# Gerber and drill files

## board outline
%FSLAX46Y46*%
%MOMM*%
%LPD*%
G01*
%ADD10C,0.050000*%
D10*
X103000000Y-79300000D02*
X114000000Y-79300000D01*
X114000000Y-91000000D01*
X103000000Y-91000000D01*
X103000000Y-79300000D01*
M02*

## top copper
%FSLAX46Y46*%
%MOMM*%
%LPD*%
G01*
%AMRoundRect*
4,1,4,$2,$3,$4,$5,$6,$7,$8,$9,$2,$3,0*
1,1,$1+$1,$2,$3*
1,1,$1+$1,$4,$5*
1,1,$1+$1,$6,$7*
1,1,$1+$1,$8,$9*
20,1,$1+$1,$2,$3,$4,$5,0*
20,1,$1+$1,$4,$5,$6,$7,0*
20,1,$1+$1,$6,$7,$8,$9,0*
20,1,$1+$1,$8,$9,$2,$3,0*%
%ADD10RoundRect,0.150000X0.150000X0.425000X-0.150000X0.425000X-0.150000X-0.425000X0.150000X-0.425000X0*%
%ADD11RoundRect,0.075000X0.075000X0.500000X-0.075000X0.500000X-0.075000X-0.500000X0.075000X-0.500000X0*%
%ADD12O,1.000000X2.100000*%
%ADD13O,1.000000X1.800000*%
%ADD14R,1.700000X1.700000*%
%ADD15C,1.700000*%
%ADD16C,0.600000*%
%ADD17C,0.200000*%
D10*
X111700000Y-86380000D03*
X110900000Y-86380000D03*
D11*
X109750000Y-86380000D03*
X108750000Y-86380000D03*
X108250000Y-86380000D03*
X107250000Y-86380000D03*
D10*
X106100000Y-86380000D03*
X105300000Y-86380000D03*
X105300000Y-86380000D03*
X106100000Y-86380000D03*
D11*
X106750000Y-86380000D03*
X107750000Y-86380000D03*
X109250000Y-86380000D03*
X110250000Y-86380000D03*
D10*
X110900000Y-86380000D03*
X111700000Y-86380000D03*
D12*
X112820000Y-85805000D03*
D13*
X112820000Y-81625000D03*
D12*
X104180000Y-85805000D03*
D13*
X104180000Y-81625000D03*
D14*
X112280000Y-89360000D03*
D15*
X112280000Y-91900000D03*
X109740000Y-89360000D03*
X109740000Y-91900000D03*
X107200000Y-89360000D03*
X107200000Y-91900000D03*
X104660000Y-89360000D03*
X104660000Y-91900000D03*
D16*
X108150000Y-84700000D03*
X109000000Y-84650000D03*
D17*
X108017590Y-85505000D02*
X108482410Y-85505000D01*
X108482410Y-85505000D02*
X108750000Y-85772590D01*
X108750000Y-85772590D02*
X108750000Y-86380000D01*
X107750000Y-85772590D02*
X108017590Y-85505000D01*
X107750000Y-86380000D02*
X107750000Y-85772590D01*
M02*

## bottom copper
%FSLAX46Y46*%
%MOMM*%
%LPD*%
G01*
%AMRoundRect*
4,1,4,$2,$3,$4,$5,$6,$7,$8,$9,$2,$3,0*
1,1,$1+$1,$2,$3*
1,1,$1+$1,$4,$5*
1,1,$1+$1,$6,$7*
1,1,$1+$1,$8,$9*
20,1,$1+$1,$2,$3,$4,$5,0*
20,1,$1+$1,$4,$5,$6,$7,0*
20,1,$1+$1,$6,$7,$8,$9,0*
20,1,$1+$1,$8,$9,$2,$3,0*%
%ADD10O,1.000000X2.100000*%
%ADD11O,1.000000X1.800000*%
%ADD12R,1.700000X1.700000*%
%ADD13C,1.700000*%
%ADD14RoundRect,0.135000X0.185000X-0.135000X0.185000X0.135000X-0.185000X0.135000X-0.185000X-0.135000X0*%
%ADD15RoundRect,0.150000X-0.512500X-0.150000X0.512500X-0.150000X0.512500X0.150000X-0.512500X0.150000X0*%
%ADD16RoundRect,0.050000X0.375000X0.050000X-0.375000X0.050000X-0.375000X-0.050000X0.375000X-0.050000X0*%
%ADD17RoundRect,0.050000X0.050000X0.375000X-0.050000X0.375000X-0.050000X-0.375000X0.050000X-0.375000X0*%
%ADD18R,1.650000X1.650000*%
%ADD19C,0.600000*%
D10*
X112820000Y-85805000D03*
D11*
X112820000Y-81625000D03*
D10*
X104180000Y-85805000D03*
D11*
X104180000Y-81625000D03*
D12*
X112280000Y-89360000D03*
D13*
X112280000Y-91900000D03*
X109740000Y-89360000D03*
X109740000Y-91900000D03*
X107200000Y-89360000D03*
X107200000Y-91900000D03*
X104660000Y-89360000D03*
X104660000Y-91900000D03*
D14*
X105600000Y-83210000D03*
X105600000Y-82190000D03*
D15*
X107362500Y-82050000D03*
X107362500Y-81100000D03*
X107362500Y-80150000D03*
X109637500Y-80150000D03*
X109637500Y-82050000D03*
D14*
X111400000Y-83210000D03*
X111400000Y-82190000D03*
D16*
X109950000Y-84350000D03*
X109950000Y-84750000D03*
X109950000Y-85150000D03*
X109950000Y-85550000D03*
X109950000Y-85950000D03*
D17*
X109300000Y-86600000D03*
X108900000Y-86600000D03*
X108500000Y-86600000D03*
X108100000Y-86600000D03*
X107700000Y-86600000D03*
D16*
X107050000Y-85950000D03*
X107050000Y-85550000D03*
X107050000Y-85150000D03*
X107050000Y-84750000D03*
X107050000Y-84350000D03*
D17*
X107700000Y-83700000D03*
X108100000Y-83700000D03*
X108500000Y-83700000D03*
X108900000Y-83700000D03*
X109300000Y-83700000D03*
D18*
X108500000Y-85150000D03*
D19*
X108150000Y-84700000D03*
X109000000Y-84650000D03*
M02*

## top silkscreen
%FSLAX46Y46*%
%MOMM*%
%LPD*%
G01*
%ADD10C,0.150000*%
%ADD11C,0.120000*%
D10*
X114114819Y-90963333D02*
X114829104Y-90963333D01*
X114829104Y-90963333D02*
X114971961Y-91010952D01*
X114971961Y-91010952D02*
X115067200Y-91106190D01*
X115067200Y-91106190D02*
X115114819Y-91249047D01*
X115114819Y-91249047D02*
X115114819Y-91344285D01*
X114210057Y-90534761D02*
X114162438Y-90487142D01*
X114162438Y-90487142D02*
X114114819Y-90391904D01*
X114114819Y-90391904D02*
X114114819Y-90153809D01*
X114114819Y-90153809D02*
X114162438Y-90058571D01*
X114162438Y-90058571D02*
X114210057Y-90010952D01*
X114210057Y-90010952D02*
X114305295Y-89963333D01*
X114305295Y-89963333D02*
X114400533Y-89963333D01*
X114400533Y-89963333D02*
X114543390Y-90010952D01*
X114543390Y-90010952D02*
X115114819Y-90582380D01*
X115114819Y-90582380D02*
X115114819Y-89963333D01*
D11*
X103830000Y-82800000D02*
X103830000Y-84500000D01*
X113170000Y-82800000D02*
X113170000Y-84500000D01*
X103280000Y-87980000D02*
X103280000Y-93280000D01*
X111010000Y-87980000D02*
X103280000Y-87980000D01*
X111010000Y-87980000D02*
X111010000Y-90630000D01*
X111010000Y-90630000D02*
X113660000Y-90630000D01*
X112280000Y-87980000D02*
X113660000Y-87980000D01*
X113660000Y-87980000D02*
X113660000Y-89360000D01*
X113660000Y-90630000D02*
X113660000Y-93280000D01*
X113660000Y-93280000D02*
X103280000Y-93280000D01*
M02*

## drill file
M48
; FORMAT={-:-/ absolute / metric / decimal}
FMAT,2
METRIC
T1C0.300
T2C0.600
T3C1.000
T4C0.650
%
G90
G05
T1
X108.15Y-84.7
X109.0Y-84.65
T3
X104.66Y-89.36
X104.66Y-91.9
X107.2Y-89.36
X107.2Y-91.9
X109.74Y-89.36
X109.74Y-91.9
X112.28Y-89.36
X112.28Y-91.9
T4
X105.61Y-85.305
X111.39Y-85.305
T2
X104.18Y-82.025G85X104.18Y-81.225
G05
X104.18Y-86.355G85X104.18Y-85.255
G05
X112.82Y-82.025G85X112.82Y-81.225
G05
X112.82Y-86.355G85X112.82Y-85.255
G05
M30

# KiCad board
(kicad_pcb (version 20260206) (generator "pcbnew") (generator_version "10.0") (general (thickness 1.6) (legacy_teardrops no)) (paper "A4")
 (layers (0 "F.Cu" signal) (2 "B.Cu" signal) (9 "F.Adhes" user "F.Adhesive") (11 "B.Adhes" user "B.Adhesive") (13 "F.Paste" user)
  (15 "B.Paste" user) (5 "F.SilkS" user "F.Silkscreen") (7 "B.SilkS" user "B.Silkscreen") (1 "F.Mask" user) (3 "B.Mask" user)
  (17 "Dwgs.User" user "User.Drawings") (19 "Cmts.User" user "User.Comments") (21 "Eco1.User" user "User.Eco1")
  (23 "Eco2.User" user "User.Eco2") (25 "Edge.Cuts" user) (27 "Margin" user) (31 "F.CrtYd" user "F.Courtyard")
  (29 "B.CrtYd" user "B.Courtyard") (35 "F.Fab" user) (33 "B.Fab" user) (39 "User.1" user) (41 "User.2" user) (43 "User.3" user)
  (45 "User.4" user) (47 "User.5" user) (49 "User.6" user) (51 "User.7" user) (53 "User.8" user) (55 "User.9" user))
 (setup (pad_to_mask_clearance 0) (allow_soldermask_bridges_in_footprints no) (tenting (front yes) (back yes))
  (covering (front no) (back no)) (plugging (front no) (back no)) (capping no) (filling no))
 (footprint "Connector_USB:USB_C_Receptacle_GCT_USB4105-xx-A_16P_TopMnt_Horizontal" (layer "F.Cu") (at 108.5 82.7 180)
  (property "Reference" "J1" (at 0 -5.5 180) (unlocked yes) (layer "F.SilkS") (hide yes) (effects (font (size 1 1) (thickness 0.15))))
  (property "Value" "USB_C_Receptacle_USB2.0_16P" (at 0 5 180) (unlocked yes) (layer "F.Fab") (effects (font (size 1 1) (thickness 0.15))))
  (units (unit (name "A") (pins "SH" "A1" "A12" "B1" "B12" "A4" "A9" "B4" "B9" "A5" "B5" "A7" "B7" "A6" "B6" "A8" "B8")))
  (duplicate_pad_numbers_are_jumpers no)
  (fp_line (start 4.67 -0.1) (end 4.67 -1.8) (stroke (width 0.12) (type solid)) (layer "F.SilkS"))
  (fp_line (start -4.67 -0.1) (end -4.67 -1.8) (stroke (width 0.12) (type solid)) (layer "F.SilkS"))
  (pad "" np_thru_hole circle (at -2.89 -2.605 180) (size 0.65 0.65) (drill 0.65) (layers "*.Cu" "*.Mask"))
  (pad "" np_thru_hole circle (at 2.89 -2.605 180) (size 0.65 0.65) (drill 0.65) (layers "*.Cu" "*.Mask"))
  (pad "A1" smd roundrect (at -3.2 -3.68 180) (size 0.6 1.15) (layers "F.Cu" "F.Mask" "F.Paste") (roundrect_rratio 0.25) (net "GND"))
  (pad "A4" smd roundrect (at -2.4 -3.68 180) (size 0.6 1.15) (layers "F.Cu" "F.Mask" "F.Paste") (roundrect_rratio 0.25) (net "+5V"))
  (pad "A5" smd roundrect (at -1.25 -3.68 180) (size 0.3 1.15) (layers "F.Cu" "F.Mask" "F.Paste") (roundrect_rratio 0.25)
   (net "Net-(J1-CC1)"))
  (pad "A6" smd roundrect (at -0.25 -3.68 180) (size 0.3 1.15) (layers "F.Cu" "F.Mask" "F.Paste") (roundrect_rratio 0.25) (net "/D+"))
  (pad "A7" smd roundrect (at 0.25 -3.68 180) (size 0.3 1.15) (layers "F.Cu" "F.Mask" "F.Paste") (roundrect_rratio 0.25) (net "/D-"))
  (pad "A8" smd roundrect (at 1.25 -3.68 180) (size 0.3 1.15) (layers "F.Cu" "F.Mask" "F.Paste") (roundrect_rratio 0.25)
   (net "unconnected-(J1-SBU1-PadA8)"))
  (pad "A9" smd roundrect (at 2.4 -3.68 180) (size 0.6 1.15) (layers "F.Cu" "F.Mask" "F.Paste") (roundrect_rratio 0.25) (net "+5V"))
  (pad "A12" smd roundrect (at 3.2 -3.68 180) (size 0.6 1.15) (layers "F.Cu" "F.Mask" "F.Paste") (roundrect_rratio 0.25) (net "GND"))
  (pad "B1" smd roundrect (at 3.2 -3.68 180) (size 0.6 1.15) (layers "F.Cu" "F.Mask" "F.Paste") (roundrect_rratio 0.25) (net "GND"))
  (pad "B4" smd roundrect (at 2.4 -3.68 180) (size 0.6 1.15) (layers "F.Cu" "F.Mask" "F.Paste") (roundrect_rratio 0.25) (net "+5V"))
  (pad "B5" smd roundrect (at 1.75 -3.68 180) (size 0.3 1.15) (layers "F.Cu" "F.Mask" "F.Paste") (roundrect_rratio 0.25)
   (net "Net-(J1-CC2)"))
  (pad "B6" smd roundrect (at 0.75 -3.68 180) (size 0.3 1.15) (layers "F.Cu" "F.Mask" "F.Paste") (roundrect_rratio 0.25) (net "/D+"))
  (pad "B7" smd roundrect (at -0.75 -3.68 180) (size 0.3 1.15) (layers "F.Cu" "F.Mask" "F.Paste") (roundrect_rratio 0.25) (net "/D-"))
  (pad "B8" smd roundrect (at -1.75 -3.68 180) (size 0.3 1.15) (layers "F.Cu" "F.Mask" "F.Paste") (roundrect_rratio 0.25)
   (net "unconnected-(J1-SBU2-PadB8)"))
  (pad "B9" smd roundrect (at -2.4 -3.68 180) (size 0.6 1.15) (layers "F.Cu" "F.Mask" "F.Paste") (roundrect_rratio 0.25) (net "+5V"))
  (pad "B12" smd roundrect (at -3.2 -3.68 180) (size 0.6 1.15) (layers "F.Cu" "F.Mask" "F.Paste") (roundrect_rratio 0.25) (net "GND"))
  (pad "SH" thru_hole oval (at -4.32 -3.105 180) (size 1 2.1) (drill oval 0.6 1.7) (layers "*.Cu" "*.Mask" "F.Paste")
   (remove_unused_layers no) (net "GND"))
  (pad "SH" thru_hole oval (at -4.32 1.075 180) (size 1 1.8) (drill oval 0.6 1.4) (layers "*.Cu" "*.Mask" "F.Paste")
   (remove_unused_layers no) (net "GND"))
  (pad "SH" thru_hole oval (at 4.32 -3.105 180) (size 1 2.1) (drill oval 0.6 1.7) (layers "*.Cu" "*.Mask" "F.Paste")
   (remove_unused_layers no) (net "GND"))
  (pad "SH" thru_hole oval (at 4.32 1.075 180) (size 1 1.8) (drill oval 0.6 1.4) (layers "*.Cu" "*.Mask" "F.Paste")
   (remove_unused_layers no) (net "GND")))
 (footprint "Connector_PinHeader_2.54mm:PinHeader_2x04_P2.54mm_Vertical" (layer "F.Cu") (at 112.28 89.36 -90)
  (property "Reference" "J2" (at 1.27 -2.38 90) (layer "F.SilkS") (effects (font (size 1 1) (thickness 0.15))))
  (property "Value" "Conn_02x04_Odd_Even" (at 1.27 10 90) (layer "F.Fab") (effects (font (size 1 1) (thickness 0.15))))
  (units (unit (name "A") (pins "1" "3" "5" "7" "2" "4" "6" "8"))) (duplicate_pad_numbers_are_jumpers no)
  (fp_line (start -1.38 9) (end 3.92 9) (stroke (width 0.12) (type solid)) (layer "F.SilkS"))
  (fp_line (start -1.38 1.27) (end -1.38 9) (stroke (width 0.12) (type solid)) (layer "F.SilkS"))
  (fp_line (start -1.38 1.27) (end 1.27 1.27) (stroke (width 0.12) (type solid)) (layer "F.SilkS"))
  (fp_line (start 1.27 1.27) (end 1.27 -1.38) (stroke (width 0.12) (type solid)) (layer "F.SilkS"))
  (fp_line (start -1.38 0) (end -1.38 -1.38) (stroke (width 0.12) (type solid)) (layer "F.SilkS"))
  (fp_line (start -1.38 -1.38) (end 0 -1.38) (stroke (width 0.12) (type solid)) (layer "F.SilkS"))
  (fp_line (start 1.27 -1.38) (end 3.92 -1.38) (stroke (width 0.12) (type solid)) (layer "F.SilkS"))
  (fp_line (start 3.92 -1.38) (end 3.92 9) (stroke (width 0.12) (type solid)) (layer "F.SilkS"))
  (pad "1" thru_hole rect (at 0 0 270) (size 1.7 1.7) (drill 1) (layers "*.Cu" "*.Mask") (remove_unused_layers no) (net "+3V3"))
  (pad "2" thru_hole circle (at 2.54 0 270) (size 1.7 1.7) (drill 1) (layers "*.Cu" "*.Mask") (remove_unused_layers no) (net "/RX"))
  (pad "3" thru_hole circle (at 0 2.54 270) (size 1.7 1.7) (drill 1) (layers "*.Cu" "*.Mask") (remove_unused_layers no) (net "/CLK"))
  (pad "4" thru_hole circle (at 2.54 2.54 270) (size 1.7 1.7) (drill 1) (layers "*.Cu" "*.Mask") (remove_unused_layers no) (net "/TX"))
  (pad "5" thru_hole circle (at 0 5.08 270) (size 1.7 1.7) (drill 1) (layers "*.Cu" "*.Mask") (remove_unused_layers no) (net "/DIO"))
  (pad "6" thru_hole circle (at 2.54 5.08 270) (size 1.7 1.7) (drill 1) (layers "*.Cu" "*.Mask") (remove_unused_layers no) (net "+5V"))
  (pad "7" thru_hole circle (at 0 7.62 270) (size 1.7 1.7) (drill 1) (layers "*.Cu" "*.Mask") (remove_unused_layers no) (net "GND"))
  (pad "8" thru_hole circle (at 2.54 7.62 270) (size 1.7 1.7) (drill 1) (layers "*.Cu" "*.Mask") (remove_unused_layers no) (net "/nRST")))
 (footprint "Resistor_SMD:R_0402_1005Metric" (layer "B.Cu") (at 105.6 82.7 90)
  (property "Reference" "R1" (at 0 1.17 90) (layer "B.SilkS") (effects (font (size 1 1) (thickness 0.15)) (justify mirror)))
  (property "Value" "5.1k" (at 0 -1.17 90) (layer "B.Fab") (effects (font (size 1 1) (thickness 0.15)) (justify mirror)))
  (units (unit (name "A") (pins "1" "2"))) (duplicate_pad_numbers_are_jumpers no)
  (pad "1" smd roundrect (at -0.51 0 90) (size 0.54 0.64) (layers "B.Cu" "B.Mask" "B.Paste") (roundrect_rratio 0.25) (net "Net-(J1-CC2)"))
  (pad "2" smd roundrect (at 0.51 0 90) (size 0.54 0.64) (layers "B.Cu" "B.Mask" "B.Paste") (roundrect_rratio 0.25) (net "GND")))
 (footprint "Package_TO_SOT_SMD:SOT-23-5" (layer "B.Cu") (at 108.5 81.1)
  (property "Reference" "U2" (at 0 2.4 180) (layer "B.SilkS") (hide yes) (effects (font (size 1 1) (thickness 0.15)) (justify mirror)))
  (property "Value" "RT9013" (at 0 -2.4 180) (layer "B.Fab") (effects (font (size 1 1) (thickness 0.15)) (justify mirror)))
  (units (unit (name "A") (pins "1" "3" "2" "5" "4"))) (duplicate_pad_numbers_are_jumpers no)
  (pad "1" smd roundrect (at -1.1375 0.95) (size 1.325 0.6) (layers "B.Cu" "B.Mask" "B.Paste") (roundrect_rratio 0.25) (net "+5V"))
  (pad "2" smd roundrect (at -1.1375 0) (size 1.325 0.6) (layers "B.Cu" "B.Mask" "B.Paste") (roundrect_rratio 0.25) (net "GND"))
  (pad "3" smd roundrect (at -1.1375 -0.95) (size 1.325 0.6) (layers "B.Cu" "B.Mask" "B.Paste") (roundrect_rratio 0.25) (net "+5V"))
  (pad "4" smd roundrect (at 1.1375 -0.95) (size 1.325 0.6) (layers "B.Cu" "B.Mask" "B.Paste") (roundrect_rratio 0.25)
   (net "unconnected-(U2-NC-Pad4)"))
  (pad "5" smd roundrect (at 1.1375 0.95) (size 1.325 0.6) (layers "B.Cu" "B.Mask" "B.Paste") (roundrect_rratio 0.25) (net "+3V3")))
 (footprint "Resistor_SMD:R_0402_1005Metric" (layer "B.Cu") (at 111.4 82.7 90)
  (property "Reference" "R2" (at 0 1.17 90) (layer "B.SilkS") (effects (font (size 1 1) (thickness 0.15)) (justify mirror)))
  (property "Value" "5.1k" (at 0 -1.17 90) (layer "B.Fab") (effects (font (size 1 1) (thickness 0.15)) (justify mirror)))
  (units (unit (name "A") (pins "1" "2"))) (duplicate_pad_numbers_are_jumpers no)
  (pad "1" smd roundrect (at -0.51 0 90) (size 0.54 0.64) (layers "B.Cu" "B.Mask" "B.Paste") (roundrect_rratio 0.25) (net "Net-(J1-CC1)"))
  (pad "2" smd roundrect (at 0.51 0 90) (size 0.54 0.64) (layers "B.Cu" "B.Mask" "B.Paste") (roundrect_rratio 0.25) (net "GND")))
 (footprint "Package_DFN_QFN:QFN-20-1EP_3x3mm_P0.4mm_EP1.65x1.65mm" (layer "B.Cu") (at 108.5 85.15 180)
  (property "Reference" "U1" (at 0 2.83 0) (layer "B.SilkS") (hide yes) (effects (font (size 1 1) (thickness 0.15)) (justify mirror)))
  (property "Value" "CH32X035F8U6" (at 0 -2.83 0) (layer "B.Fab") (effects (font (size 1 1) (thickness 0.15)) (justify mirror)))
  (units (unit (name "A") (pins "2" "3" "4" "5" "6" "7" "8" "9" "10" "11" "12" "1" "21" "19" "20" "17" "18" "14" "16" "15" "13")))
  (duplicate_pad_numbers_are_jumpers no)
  (pad "" smd roundrect (at -0.41 -0.41 180) (size 0.67 0.67) (layers "B.Paste") (roundrect_rratio 0.25))
  (pad "" smd roundrect (at -0.41 0.41 180) (size 0.67 0.67) (layers "B.Paste") (roundrect_rratio 0.25))
  (pad "" smd roundrect (at 0.41 -0.41 180) (size 0.67 0.67) (layers "B.Paste") (roundrect_rratio 0.25))
  (pad "" smd roundrect (at 0.41 0.41 180) (size 0.67 0.67) (layers "B.Paste") (roundrect_rratio 0.25))
  (pad "1" smd roundrect (at -1.45 0.8 180) (size 0.85 0.2) (layers "B.Cu" "B.Mask" "B.Paste") (roundrect_rratio 0.25)
   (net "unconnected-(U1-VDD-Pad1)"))
  (pad "2" smd roundrect (at -1.45 0.4 180) (size 0.85 0.2) (layers "B.Cu" "B.Mask" "B.Paste") (roundrect_rratio 0.25)
   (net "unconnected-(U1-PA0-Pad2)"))
  (pad "3" smd roundrect (at -1.45 0 180) (size 0.85 0.2) (layers "B.Cu" "B.Mask" "B.Paste") (roundrect_rratio 0.25)
   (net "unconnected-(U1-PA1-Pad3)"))
  (pad "4" smd roundrect (at -1.45 -0.4 180) (size 0.85 0.2) (layers "B.Cu" "B.Mask" "B.Paste") (roundrect_rratio 0.25)
   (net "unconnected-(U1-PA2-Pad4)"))
  (pad "5" smd roundrect (at -1.45 -0.8 180) (size 0.85 0.2) (layers "B.Cu" "B.Mask" "B.Paste") (roundrect_rratio 0.25)
   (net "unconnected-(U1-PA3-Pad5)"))
  (pad "6" smd roundrect (at -0.8 -1.45 180) (size 0.2 0.85) (layers "B.Cu" "B.Mask" "B.Paste") (roundrect_rratio 0.25)
   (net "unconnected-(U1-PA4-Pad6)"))
  (pad "7" smd roundrect (at -0.4 -1.45 180) (size 0.2 0.85) (layers "B.Cu" "B.Mask" "B.Paste") (roundrect_rratio 0.25)
   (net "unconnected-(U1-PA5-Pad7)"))
  (pad "8" smd roundrect (at 0 -1.45 180) (size 0.2 0.85) (layers "B.Cu" "B.Mask" "B.Paste") (roundrect_rratio 0.25)
   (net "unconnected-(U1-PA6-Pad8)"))
  (pad "9" smd roundrect (at 0.4 -1.45 180) (size 0.2 0.85) (layers "B.Cu" "B.Mask" "B.Paste") (roundrect_rratio 0.25)
   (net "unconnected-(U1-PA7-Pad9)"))
  (pad "10" smd roundrect (at 0.8 -1.45 180) (size 0.2 0.85) (layers "B.Cu" "B.Mask" "B.Paste") (roundrect_rratio 0.25)
   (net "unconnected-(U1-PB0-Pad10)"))
  (pad "11" smd roundrect (at 1.45 -0.8 180) (size 0.85 0.2) (layers "B.Cu" "B.Mask" "B.Paste") (roundrect_rratio 0.25)
   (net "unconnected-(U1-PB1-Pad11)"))
  (pad "12" smd roundrect (at 1.45 -0.4 180) (size 0.85 0.2) (layers "B.Cu" "B.Mask" "B.Paste") (roundrect_rratio 0.25)
   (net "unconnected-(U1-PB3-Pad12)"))
  (pad "13" smd roundrect (at 1.45 0 180) (size 0.85 0.2) (layers "B.Cu" "B.Mask" "B.Paste") (roundrect_rratio 0.25)
   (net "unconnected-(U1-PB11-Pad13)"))
  (pad "14" smd roundrect (at 1.45 0.4 180) (size 0.85 0.2) (layers "B.Cu" "B.Mask" "B.Paste") (roundrect_rratio 0.25)
   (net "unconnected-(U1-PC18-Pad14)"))
  (pad "15" smd roundrect (at 1.45 0.8 180) (size 0.85 0.2) (layers "B.Cu" "B.Mask" "B.Paste") (roundrect_rratio 0.25)
   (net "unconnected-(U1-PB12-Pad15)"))
  (pad "16" smd roundrect (at 0.8 1.45 180) (size 0.2 0.85) (layers "B.Cu" "B.Mask" "B.Paste") (roundrect_rratio 0.25)
   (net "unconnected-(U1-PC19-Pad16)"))
  (pad "17" smd roundrect (at 0.4 1.45 180) (size 0.2 0.85) (layers "B.Cu" "B.Mask" "B.Paste") (roundrect_rratio 0.25) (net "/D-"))
  (pad "18" smd roundrect (at 0 1.45 180) (size 0.2 0.85) (layers "B.Cu" "B.Mask" "B.Paste") (roundrect_rratio 0.25) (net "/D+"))
  (pad "19" smd roundrect (at -0.4 1.45 180) (size 0.2 0.85) (layers "B.Cu" "B.Mask" "B.Paste") (roundrect_rratio 0.25) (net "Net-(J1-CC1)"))
  (pad "20" smd roundrect (at -0.8 1.45 180) (size 0.2 0.85) (layers "B.Cu" "B.Mask" "B.Paste") (roundrect_rratio 0.25) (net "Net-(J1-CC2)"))
  (pad "21" smd rect (at 0 0 180) (size 1.65 1.65) (layers "B.Cu" "B.Mask") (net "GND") (zone_connect 2)))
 (gr_rect (start 103 79.3) (end 114 91) (stroke (width 0.05) (type default)) (fill no) (layer "Edge.Cuts"))
 (via (at 108.15 84.7) (size 0.6) (drill 0.3) (layers "F.Cu" "B.Cu") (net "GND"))
 (via (at 109 84.65) (size 0.6) (drill 0.3) (layers "F.Cu" "B.Cu") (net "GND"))
 (segment (start 108.01759 85.505) (end 108.48241 85.505) (width 0.2) (layer "F.Cu") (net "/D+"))
 (segment (start 108.48241 85.505) (end 108.75 85.77259) (width 0.2) (layer "F.Cu") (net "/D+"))
 (segment (start 108.75 85.77259) (end 108.75 86.38) (width 0.2) (layer "F.Cu") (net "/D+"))
 (segment (start 107.75 85.77259) (end 108.01759 85.505) (width 0.2) (layer "F.Cu") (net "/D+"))
 (segment (start 107.75 86.38) (end 107.75 85.77259) (width 0.2) (layer "F.Cu") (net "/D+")))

